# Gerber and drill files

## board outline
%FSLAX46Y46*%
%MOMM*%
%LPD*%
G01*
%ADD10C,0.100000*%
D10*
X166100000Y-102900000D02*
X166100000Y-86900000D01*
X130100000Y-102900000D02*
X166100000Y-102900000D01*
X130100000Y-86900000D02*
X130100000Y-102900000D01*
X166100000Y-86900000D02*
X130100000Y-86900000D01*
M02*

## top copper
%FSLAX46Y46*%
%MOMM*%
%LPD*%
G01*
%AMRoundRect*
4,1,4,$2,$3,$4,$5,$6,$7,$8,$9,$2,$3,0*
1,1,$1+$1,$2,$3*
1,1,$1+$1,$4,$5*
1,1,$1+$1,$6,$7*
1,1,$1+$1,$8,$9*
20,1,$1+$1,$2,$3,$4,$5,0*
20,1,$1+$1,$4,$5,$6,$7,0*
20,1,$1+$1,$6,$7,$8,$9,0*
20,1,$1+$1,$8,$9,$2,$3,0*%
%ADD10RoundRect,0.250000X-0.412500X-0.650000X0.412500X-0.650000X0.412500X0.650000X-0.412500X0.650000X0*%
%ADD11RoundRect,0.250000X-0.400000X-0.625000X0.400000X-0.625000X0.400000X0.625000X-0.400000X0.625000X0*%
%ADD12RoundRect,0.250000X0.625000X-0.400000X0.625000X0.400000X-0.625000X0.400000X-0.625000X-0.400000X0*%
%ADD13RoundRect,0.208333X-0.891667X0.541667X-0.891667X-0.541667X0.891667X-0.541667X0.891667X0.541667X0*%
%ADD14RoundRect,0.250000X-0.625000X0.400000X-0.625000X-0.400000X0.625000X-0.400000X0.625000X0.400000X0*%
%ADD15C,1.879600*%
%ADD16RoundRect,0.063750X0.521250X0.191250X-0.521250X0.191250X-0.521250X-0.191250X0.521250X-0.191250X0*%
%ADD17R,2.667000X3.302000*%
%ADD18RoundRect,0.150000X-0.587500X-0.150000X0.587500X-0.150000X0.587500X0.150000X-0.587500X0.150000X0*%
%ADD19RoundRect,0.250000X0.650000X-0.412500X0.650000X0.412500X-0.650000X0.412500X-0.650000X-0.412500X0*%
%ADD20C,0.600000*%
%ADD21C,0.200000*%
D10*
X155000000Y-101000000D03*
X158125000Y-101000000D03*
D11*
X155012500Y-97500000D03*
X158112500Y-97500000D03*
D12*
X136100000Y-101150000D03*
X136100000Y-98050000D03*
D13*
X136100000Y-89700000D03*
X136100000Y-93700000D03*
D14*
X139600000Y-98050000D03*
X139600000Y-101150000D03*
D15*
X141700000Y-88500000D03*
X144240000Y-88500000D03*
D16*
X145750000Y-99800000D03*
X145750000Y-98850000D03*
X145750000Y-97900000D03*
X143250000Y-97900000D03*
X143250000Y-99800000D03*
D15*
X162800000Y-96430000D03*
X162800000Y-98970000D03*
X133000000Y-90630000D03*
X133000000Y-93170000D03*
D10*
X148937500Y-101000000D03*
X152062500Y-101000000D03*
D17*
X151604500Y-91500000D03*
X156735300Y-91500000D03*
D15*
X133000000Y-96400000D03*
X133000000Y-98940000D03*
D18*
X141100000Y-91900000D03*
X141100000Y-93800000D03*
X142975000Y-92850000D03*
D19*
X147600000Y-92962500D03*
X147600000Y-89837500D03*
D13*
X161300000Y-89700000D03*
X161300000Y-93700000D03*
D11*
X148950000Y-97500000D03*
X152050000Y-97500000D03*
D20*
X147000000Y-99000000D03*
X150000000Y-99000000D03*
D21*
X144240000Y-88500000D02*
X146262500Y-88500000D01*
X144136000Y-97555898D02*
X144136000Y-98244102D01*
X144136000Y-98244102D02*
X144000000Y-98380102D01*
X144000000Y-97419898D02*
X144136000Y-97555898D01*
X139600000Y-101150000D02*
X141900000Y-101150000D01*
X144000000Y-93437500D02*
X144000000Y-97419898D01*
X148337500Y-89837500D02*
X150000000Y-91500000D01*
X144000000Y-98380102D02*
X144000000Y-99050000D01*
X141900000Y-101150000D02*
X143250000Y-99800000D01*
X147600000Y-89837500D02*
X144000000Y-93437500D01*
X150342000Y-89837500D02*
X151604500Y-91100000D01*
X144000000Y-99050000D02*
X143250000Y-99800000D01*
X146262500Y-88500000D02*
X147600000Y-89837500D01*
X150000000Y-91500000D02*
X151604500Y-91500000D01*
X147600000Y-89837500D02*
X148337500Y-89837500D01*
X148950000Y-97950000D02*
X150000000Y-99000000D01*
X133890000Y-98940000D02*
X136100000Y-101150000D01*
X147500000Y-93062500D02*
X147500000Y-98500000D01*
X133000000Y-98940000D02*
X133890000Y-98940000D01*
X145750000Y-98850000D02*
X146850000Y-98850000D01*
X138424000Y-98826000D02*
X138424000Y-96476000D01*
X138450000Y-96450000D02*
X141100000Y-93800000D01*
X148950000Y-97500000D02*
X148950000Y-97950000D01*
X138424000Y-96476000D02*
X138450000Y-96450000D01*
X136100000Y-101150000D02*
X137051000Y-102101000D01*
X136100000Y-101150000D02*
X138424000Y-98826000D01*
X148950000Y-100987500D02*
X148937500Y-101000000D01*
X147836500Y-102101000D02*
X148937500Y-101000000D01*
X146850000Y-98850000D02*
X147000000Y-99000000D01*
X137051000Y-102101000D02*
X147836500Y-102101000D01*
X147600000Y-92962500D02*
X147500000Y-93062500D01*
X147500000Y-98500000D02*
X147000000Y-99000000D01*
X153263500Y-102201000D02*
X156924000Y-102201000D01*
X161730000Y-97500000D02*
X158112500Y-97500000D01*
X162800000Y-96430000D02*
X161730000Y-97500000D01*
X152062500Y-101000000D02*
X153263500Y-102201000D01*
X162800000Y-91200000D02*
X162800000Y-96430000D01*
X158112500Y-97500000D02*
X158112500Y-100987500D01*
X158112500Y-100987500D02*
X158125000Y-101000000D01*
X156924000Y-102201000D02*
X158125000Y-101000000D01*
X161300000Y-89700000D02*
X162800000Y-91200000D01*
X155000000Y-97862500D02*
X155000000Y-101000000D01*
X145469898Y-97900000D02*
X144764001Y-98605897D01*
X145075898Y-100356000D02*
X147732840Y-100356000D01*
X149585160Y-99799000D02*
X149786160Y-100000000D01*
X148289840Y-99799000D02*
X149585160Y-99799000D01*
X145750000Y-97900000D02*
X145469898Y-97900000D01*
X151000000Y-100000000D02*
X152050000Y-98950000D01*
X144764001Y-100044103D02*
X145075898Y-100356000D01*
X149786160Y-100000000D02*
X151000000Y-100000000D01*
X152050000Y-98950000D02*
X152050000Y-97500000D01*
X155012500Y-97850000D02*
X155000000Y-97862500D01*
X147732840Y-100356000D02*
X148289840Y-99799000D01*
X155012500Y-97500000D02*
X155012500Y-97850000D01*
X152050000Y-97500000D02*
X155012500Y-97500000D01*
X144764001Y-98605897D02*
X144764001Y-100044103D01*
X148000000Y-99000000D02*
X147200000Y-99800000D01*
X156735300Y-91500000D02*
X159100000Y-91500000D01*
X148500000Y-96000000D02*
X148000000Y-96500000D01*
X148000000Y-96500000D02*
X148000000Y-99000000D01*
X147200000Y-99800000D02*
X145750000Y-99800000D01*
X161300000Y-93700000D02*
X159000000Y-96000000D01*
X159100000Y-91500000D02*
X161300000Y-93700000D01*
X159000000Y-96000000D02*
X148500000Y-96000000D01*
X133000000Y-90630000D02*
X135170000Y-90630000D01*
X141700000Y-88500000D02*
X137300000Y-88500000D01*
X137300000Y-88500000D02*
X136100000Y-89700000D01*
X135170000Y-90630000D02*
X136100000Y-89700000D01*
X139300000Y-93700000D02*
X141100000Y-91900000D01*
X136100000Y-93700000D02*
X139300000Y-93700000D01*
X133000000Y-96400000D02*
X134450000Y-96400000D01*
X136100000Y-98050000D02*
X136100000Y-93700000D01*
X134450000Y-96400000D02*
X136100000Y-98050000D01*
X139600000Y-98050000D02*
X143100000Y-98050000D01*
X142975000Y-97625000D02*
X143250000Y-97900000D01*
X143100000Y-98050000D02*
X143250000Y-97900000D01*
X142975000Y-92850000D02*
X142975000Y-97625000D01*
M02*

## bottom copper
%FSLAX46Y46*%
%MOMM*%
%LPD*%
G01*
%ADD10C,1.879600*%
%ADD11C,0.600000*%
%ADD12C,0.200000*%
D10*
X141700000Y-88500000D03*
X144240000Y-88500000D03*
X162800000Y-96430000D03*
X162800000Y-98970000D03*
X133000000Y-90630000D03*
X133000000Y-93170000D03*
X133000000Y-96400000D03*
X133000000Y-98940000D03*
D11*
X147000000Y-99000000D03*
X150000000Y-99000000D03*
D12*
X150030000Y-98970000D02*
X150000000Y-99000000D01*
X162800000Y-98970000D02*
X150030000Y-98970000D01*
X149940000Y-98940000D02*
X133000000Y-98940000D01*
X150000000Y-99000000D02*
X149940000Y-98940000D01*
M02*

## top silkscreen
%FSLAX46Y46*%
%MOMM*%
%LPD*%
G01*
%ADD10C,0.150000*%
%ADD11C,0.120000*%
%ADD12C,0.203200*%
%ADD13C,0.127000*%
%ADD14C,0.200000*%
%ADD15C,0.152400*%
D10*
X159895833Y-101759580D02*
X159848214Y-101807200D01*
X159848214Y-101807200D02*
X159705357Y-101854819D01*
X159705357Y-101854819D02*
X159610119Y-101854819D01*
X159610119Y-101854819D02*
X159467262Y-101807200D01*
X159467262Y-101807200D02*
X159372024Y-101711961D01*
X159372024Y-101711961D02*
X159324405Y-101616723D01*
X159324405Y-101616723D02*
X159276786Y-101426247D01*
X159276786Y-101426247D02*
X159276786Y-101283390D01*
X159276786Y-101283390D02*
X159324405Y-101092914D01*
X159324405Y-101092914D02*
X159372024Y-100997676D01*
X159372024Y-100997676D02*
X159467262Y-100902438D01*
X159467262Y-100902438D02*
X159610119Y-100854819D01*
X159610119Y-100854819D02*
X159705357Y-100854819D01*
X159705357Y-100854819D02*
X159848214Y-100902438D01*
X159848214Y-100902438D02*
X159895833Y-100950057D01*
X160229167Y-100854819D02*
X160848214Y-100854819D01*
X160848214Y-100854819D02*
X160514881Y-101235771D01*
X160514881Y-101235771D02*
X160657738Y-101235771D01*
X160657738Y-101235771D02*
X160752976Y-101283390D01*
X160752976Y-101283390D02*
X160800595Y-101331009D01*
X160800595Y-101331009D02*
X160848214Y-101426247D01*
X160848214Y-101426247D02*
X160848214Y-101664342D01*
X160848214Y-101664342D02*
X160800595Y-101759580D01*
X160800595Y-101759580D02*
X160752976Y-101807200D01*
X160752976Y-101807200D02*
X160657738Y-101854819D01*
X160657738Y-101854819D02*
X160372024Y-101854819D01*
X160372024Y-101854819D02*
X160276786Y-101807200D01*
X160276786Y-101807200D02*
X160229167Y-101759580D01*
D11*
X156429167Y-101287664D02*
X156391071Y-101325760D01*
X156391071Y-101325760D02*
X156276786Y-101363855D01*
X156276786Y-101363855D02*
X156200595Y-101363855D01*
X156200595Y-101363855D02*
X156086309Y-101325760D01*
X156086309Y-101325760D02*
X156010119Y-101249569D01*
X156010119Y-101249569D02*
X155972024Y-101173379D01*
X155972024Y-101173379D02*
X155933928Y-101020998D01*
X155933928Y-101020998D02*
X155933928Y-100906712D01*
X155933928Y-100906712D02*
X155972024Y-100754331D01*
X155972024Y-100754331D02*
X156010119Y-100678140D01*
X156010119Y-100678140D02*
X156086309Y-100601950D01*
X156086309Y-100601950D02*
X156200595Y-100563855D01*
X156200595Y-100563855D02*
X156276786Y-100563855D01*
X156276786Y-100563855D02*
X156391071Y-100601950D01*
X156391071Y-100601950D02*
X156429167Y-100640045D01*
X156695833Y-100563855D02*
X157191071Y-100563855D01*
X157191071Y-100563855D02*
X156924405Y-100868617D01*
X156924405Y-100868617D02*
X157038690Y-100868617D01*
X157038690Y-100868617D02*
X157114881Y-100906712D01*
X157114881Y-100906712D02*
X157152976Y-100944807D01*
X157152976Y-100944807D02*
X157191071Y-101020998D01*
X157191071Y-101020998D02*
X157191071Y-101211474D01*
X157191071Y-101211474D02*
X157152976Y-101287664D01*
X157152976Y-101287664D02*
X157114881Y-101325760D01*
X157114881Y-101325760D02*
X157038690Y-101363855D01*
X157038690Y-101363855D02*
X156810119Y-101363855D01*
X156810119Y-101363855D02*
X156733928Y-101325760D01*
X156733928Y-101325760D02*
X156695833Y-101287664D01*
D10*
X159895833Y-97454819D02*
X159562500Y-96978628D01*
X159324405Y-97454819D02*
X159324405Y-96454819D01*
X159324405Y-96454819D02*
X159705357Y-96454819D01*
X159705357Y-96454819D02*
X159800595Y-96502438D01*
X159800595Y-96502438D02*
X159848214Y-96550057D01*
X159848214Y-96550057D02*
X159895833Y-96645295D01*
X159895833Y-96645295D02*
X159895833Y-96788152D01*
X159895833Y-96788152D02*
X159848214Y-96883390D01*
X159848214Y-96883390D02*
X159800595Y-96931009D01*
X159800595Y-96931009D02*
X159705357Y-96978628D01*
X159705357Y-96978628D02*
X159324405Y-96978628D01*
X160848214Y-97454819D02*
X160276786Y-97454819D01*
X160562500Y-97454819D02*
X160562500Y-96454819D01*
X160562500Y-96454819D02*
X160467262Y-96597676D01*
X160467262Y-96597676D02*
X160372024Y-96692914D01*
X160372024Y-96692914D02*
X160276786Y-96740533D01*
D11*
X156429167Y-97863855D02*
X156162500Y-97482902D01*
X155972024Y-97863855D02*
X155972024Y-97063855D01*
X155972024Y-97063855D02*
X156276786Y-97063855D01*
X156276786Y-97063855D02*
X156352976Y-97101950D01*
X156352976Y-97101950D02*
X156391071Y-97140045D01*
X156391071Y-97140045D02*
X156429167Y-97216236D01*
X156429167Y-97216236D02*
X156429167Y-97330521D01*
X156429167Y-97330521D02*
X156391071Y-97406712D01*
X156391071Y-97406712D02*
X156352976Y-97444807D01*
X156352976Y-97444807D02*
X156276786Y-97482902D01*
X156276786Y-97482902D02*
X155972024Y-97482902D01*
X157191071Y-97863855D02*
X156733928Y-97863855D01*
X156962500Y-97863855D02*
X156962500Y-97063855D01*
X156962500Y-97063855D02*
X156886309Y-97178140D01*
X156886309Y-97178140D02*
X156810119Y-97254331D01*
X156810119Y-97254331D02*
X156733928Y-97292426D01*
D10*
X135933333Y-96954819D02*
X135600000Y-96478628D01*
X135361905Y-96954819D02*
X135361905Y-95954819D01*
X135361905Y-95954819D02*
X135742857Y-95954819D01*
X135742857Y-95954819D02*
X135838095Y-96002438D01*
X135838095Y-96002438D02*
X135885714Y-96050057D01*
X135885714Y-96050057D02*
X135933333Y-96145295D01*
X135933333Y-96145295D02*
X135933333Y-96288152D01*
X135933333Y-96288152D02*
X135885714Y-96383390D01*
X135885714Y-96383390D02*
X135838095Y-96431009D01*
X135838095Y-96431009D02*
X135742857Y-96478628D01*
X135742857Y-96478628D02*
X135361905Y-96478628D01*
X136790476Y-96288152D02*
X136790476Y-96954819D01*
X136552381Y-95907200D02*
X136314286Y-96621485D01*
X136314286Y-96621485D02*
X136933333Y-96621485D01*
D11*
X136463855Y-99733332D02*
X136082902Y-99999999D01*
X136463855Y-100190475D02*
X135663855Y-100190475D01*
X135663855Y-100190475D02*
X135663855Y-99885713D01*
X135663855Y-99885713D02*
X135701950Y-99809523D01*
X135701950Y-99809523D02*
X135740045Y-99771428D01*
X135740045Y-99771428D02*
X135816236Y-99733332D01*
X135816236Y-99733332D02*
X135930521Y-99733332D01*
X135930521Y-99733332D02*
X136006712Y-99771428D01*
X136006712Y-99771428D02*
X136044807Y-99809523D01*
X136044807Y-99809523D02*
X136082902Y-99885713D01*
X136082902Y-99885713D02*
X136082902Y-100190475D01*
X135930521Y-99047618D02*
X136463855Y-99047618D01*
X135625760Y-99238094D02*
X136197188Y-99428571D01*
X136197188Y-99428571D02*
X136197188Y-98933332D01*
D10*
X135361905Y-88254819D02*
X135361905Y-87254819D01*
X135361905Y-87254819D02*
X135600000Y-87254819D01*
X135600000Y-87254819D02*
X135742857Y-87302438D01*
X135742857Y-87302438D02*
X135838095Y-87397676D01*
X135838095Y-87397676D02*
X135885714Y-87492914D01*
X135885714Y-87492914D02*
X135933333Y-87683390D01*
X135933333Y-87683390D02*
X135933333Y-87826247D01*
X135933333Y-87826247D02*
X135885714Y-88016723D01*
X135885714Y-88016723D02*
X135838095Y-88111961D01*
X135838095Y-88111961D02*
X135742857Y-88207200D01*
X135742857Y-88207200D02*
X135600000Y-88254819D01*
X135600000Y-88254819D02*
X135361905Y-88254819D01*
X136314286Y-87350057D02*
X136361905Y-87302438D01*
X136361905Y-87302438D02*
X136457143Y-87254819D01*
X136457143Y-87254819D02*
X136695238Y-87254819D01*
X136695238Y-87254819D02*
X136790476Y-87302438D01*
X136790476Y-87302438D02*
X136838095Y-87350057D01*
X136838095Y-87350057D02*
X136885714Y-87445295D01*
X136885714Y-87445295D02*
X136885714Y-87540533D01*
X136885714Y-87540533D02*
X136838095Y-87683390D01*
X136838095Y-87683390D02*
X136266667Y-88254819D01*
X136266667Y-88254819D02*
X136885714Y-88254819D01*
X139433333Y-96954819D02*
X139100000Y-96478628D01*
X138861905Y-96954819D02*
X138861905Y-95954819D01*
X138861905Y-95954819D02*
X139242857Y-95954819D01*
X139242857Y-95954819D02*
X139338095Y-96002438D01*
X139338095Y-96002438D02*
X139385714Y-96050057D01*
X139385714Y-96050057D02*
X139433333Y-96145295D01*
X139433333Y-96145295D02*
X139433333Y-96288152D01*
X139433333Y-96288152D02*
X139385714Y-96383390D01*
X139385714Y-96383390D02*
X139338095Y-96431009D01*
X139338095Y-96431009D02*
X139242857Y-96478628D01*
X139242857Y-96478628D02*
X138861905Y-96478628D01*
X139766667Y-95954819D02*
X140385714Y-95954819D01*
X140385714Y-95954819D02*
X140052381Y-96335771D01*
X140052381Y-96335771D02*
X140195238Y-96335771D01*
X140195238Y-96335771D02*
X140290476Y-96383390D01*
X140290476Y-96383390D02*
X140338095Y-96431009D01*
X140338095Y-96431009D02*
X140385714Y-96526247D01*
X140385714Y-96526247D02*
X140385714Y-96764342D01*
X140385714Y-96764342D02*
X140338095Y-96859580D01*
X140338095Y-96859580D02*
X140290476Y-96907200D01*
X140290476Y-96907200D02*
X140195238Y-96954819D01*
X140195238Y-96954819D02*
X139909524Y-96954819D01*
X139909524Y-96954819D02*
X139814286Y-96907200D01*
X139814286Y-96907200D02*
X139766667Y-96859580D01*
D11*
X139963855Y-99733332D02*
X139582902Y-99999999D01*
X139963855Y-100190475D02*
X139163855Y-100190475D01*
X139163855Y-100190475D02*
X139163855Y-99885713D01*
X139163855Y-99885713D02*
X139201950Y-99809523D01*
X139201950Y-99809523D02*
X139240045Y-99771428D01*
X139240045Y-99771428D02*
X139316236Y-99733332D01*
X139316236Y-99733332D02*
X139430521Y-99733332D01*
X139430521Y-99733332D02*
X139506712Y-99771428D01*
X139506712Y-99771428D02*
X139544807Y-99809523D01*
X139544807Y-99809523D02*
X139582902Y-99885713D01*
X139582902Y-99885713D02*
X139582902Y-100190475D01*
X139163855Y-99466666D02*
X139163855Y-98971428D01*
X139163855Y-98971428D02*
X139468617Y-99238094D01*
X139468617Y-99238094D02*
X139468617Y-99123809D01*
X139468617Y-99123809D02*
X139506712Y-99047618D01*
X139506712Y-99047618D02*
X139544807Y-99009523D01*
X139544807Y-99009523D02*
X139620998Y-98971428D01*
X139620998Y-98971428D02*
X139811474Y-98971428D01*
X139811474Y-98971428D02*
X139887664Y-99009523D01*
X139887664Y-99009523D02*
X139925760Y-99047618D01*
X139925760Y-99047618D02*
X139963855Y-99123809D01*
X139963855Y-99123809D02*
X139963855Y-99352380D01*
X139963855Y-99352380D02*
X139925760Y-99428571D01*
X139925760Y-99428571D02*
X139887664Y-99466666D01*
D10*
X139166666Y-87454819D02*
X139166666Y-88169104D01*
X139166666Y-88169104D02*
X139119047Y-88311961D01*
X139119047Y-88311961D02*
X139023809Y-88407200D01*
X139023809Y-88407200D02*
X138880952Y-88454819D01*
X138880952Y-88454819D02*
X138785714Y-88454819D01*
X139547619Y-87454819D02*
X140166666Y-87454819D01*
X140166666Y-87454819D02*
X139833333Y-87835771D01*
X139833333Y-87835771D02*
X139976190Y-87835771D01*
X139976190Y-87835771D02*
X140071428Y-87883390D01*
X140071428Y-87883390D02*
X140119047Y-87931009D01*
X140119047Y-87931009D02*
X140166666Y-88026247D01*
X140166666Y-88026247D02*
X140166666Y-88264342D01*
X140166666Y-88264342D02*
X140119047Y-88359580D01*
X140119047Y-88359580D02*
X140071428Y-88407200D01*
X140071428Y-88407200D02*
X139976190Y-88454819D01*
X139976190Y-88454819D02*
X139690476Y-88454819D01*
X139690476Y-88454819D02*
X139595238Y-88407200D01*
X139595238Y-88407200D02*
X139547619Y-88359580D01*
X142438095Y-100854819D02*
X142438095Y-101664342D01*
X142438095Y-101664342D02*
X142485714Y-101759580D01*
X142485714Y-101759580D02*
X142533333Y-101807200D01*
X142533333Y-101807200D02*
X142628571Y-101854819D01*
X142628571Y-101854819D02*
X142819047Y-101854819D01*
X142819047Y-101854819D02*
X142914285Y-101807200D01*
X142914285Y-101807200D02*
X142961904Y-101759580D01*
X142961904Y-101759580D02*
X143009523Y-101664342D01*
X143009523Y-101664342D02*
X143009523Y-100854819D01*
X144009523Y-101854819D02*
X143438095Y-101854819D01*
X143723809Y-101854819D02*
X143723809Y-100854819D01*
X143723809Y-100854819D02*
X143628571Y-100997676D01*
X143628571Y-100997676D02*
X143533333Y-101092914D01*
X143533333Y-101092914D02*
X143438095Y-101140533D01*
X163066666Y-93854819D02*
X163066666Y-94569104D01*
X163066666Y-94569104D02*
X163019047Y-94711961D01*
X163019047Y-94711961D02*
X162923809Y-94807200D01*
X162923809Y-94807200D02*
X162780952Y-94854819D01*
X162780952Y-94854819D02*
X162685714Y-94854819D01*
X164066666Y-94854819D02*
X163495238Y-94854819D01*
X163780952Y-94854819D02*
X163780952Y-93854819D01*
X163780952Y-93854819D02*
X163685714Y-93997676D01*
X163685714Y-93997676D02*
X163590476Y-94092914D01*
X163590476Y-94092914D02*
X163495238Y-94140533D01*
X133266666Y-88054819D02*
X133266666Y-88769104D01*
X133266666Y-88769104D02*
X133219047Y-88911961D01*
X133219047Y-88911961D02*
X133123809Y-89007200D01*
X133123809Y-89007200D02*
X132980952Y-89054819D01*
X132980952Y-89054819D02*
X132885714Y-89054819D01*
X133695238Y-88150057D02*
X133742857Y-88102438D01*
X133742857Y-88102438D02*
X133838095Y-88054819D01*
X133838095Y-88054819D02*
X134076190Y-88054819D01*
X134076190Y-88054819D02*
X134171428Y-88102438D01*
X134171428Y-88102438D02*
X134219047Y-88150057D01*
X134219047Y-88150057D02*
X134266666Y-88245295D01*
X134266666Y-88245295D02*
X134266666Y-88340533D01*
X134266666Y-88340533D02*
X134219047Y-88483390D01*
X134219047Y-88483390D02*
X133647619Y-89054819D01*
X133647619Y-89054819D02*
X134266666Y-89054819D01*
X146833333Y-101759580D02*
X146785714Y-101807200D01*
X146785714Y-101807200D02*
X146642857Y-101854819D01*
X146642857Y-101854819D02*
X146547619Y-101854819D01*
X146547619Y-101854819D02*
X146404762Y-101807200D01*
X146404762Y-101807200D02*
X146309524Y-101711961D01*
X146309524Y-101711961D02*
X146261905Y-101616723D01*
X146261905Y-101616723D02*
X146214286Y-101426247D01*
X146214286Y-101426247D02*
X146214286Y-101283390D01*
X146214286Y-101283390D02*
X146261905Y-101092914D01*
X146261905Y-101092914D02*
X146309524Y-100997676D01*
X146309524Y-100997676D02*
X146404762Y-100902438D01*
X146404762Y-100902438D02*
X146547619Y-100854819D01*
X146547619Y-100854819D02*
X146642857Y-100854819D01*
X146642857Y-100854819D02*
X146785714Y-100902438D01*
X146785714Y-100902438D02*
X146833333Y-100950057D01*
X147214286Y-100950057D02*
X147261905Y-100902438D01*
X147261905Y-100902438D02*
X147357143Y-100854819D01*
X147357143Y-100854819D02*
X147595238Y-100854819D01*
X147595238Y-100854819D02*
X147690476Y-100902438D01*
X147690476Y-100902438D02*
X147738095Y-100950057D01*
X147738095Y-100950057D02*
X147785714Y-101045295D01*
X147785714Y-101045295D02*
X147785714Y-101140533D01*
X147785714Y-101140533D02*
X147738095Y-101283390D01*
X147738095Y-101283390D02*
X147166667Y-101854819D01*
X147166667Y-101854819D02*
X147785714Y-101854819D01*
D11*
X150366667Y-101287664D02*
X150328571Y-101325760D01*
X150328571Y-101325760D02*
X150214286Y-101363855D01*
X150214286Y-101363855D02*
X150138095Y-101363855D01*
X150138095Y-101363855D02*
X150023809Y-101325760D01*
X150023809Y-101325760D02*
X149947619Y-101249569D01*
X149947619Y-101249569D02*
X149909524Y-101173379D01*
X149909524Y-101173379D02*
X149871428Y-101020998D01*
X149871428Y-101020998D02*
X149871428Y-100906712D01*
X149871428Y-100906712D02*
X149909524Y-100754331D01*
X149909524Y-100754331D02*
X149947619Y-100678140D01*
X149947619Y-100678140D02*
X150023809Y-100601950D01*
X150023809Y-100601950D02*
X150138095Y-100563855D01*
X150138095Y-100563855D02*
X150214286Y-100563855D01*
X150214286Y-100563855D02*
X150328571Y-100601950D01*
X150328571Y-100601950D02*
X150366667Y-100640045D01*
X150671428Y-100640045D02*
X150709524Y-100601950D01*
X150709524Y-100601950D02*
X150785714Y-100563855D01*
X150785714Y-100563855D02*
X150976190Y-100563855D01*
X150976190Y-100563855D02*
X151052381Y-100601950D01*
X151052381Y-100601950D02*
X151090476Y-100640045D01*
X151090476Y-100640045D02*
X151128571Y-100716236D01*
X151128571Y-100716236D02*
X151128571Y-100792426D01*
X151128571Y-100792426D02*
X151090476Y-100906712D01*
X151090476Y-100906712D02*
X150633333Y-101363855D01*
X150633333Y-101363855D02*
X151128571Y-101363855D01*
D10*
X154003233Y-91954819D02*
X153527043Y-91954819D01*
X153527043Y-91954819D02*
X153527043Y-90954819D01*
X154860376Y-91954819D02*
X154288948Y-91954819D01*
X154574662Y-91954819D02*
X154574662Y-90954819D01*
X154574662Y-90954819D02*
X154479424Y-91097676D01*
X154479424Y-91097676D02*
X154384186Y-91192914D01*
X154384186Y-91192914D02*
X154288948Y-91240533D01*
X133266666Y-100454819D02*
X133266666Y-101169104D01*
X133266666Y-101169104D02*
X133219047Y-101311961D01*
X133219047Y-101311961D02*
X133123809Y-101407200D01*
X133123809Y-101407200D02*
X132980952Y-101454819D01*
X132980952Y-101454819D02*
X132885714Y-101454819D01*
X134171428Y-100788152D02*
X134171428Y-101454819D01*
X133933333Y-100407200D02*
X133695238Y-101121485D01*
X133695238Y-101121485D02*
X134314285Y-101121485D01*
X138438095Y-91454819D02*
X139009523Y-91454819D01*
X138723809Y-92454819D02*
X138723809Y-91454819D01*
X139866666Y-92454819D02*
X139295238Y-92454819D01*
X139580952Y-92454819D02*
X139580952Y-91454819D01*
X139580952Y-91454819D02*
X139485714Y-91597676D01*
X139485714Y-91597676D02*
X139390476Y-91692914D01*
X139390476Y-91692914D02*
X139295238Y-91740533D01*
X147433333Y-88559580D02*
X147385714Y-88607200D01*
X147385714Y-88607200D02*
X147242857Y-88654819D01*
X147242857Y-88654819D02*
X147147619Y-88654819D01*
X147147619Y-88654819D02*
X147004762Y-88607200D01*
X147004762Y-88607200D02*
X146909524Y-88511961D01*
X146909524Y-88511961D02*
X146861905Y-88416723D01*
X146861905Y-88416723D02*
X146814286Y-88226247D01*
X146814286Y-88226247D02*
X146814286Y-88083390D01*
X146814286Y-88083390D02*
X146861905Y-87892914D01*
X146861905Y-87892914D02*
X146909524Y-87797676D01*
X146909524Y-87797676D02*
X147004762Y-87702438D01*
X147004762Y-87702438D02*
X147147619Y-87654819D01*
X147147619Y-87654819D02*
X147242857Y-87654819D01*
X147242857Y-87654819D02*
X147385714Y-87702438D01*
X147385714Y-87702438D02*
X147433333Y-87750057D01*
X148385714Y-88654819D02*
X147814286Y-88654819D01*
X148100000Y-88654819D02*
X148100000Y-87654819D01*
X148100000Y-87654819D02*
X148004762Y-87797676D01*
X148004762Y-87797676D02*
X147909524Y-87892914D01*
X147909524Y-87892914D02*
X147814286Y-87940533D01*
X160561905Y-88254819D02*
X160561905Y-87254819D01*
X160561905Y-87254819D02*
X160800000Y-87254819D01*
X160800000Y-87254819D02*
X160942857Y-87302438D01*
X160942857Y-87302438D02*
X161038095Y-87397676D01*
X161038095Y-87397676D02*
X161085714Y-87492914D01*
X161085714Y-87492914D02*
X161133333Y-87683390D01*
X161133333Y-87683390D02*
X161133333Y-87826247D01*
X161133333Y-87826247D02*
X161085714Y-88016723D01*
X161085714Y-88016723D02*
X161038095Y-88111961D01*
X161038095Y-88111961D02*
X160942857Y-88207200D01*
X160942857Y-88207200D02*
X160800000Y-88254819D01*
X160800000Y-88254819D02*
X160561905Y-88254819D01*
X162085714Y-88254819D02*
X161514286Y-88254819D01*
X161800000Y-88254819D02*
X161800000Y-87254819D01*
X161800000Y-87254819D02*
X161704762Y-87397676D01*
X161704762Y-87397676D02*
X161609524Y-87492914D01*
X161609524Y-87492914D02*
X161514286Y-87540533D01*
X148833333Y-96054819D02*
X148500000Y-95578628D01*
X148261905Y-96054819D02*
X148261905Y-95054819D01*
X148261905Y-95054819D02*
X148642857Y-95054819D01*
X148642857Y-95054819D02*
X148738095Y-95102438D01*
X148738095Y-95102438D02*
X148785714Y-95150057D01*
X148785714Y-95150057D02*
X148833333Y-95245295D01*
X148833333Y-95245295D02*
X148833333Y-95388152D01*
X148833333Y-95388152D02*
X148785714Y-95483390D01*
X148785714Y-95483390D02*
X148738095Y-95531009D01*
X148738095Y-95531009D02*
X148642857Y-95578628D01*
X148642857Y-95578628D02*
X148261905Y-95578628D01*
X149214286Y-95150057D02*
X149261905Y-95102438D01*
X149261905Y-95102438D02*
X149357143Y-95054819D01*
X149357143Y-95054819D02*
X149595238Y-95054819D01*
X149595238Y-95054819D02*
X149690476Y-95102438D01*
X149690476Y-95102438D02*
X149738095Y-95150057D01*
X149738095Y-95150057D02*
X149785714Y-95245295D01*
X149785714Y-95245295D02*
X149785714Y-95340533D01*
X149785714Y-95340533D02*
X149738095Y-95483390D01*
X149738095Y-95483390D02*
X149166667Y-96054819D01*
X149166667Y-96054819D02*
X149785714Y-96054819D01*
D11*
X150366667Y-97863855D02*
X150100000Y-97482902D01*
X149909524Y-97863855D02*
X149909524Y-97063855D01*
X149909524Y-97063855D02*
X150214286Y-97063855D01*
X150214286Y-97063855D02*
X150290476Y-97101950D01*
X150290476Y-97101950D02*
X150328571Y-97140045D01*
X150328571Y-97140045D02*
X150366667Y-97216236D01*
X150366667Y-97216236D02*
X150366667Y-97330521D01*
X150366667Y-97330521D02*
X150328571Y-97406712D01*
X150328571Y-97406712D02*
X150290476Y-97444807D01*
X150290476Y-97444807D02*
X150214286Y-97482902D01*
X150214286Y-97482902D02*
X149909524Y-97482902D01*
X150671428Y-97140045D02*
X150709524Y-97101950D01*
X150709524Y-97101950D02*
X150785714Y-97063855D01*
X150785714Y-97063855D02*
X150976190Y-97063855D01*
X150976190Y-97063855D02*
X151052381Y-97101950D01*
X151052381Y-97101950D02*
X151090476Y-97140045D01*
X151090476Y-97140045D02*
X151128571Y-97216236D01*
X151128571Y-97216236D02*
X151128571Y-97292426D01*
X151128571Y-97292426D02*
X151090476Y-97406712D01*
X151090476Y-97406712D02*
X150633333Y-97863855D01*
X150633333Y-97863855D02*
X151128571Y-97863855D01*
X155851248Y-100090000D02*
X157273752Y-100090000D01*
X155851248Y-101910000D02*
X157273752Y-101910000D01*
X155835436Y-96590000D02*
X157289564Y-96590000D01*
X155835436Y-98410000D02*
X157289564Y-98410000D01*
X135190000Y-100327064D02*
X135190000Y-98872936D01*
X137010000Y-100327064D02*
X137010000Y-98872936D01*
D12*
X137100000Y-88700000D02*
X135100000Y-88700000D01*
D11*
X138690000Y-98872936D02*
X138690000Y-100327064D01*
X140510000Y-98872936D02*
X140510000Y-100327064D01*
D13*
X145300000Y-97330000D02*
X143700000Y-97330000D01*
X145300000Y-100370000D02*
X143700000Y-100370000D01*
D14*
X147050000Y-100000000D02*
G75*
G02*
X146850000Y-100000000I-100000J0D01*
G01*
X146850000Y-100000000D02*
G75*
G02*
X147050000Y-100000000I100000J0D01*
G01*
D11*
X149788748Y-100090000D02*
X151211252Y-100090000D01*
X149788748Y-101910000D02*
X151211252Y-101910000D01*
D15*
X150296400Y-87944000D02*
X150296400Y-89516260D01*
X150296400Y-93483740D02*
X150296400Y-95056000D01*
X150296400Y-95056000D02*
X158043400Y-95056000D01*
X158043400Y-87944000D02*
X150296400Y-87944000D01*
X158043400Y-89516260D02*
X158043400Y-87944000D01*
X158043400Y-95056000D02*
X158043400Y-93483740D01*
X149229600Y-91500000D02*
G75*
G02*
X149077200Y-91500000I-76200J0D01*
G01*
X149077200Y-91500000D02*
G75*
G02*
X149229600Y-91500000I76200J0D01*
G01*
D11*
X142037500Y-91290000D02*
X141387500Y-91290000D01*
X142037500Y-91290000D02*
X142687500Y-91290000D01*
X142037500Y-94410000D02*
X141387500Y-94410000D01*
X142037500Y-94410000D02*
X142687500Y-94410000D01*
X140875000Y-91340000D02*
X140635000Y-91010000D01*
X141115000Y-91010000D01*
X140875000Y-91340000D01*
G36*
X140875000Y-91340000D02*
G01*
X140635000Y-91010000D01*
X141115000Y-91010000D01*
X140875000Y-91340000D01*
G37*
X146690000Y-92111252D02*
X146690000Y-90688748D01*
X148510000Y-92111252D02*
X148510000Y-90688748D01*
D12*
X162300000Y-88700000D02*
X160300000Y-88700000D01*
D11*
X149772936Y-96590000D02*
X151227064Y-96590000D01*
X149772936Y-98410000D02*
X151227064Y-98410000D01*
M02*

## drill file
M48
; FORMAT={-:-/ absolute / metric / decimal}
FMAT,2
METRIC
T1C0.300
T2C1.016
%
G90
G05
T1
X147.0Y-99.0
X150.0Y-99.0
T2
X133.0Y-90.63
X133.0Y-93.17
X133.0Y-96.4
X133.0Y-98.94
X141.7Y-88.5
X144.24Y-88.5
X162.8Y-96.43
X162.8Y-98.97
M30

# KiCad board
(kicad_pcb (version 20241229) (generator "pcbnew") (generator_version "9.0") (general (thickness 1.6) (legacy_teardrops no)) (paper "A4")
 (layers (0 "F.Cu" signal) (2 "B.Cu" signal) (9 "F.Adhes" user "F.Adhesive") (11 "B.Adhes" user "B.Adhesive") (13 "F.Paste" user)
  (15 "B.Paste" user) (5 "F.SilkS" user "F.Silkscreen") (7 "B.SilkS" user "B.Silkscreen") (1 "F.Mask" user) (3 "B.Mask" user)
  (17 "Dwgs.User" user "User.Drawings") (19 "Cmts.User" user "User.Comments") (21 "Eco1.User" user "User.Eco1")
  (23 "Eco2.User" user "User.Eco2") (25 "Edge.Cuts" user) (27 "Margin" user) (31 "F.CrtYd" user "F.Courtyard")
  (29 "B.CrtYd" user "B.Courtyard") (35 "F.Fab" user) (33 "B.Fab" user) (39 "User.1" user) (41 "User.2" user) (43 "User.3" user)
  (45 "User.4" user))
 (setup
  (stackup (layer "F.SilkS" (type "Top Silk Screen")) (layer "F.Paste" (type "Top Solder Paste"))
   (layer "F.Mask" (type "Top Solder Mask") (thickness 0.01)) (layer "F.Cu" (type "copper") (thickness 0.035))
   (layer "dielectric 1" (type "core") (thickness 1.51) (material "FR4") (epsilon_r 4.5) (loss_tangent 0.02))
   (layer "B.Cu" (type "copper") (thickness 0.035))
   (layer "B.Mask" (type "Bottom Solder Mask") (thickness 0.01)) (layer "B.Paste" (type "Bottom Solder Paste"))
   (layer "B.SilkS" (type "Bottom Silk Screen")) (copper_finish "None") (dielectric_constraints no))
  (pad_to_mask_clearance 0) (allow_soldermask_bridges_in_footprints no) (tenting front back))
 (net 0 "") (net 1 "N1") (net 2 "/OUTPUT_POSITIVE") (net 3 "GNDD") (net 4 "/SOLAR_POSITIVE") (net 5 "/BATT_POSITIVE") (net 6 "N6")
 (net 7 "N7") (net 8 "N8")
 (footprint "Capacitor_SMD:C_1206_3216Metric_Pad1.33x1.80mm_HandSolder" (layer "F.Cu") (at 156.5625 101)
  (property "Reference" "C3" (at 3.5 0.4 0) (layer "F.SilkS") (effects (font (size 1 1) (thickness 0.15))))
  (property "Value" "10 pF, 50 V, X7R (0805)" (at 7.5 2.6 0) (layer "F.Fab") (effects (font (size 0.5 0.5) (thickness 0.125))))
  (fp_line (start -0.711252 -0.91) (end 0.711252 -0.91) (stroke (width 0.12) (type solid)) (layer "F.SilkS"))
  (fp_line (start -0.711252 0.91) (end 0.711252 0.91) (stroke (width 0.12) (type solid)) (layer "F.SilkS"))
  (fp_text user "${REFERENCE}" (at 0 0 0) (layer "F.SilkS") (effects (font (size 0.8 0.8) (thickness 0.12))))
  (pad "1" smd roundrect (at -1.5625 0) (size 1.325 1.8) (layers "F.Cu" "F.Mask" "F.Paste") (roundrect_rratio 0.188679) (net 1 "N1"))
  (pad "2" smd roundrect (at 1.5625 0) (size 1.325 1.8) (layers "F.Cu" "F.Mask" "F.Paste") (roundrect_rratio 0.188679)
   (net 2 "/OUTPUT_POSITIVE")))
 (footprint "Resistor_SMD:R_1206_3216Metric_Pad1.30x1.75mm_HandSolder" (layer "F.Cu") (at 156.5625 97.5)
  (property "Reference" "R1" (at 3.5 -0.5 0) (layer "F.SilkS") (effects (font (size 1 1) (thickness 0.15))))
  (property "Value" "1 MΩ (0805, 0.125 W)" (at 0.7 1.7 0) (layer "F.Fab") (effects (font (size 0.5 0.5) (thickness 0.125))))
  (fp_line (start -0.727064 -0.91) (end 0.727064 -0.91) (stroke (width 0.12) (type solid)) (layer "F.SilkS"))
  (fp_line (start -0.727064 0.91) (end 0.727064 0.91) (stroke (width 0.12) (type solid)) (layer "F.SilkS"))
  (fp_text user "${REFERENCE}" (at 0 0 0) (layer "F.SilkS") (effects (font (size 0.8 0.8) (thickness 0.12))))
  (pad "1" smd roundrect (at -1.55 0) (size 1.3 1.75) (layers "F.Cu" "F.Mask" "F.Paste") (roundrect_rratio 0.192308) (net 1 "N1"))
  (pad "2" smd roundrect (at 1.55 0) (size 1.3 1.75) (layers "F.Cu" "F.Mask" "F.Paste") (roundrect_rratio 0.192308)
   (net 2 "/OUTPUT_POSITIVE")))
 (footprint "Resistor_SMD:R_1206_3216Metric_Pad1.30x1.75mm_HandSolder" (layer "F.Cu") (at 136.1 99.6 90)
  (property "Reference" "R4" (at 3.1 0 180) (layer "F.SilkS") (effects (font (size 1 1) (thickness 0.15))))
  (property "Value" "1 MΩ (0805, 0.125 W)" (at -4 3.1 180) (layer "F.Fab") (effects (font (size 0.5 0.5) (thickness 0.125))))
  (fp_line (start -0.727064 -0.91) (end 0.727064 -0.91) (stroke (width 0.12) (type solid)) (layer "F.SilkS"))
  (fp_line (start -0.727064 0.91) (end 0.727064 0.91) (stroke (width 0.12) (type solid)) (layer "F.SilkS"))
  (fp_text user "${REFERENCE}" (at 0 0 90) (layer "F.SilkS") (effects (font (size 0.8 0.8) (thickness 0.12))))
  (pad "1" smd roundrect (at -1.55 0 90) (size 1.3 1.75) (layers "F.Cu" "F.Mask" "F.Paste") (roundrect_rratio 0.192308) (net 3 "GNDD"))
  (pad "2" smd roundrect (at 1.55 0 90) (size 1.3 1.75) (layers "F.Cu" "F.Mask" "F.Paste") (roundrect_rratio 0.192308)
   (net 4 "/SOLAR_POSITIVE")))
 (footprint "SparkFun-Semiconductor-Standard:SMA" (layer "F.Cu") (at 136.1 91.7 -90)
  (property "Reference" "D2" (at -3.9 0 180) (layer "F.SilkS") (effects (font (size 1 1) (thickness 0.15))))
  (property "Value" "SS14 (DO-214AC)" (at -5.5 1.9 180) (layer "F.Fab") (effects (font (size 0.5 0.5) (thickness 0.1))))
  (fp_line (start -3 -1) (end -3 1) (stroke (width 0.2032) (type solid)) (layer "F.SilkS"))
  (pad "1" smd roundrect (at -2 0 270) (size 1.5 2.2) (layers "F.Cu" "F.Mask" "F.Paste") (roundrect_rratio 0.1388888889)
   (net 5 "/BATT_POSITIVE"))
  (pad "2" smd roundrect (at 2 0 270) (size 1.5 2.2) (layers "F.Cu" "F.Mask" "F.Paste") (roundrect_rratio 0.1388888889)
   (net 4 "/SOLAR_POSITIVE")))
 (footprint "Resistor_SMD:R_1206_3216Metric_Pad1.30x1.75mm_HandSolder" (layer "F.Cu") (at 139.6 99.6 -90)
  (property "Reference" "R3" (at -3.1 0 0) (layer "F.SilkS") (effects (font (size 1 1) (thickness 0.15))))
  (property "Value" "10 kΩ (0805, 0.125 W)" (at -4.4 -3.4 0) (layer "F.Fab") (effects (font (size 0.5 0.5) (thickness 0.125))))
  (fp_line (start -0.727064 0.91) (end 0.727064 0.91) (stroke (width 0.12) (type solid)) (layer "F.SilkS"))
  (fp_line (start -0.727064 -0.91) (end 0.727064 -0.91) (stroke (width 0.12) (type solid)) (layer "F.SilkS"))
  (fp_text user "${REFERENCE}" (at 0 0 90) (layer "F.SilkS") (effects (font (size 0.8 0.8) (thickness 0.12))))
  (pad "1" smd roundrect (at -1.55 0 270) (size 1.3 1.75) (layers "F.Cu" "F.Mask" "F.Paste") (roundrect_rratio 0.192308) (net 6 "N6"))
  (pad "2" smd roundrect (at 1.55 0 270) (size 1.3 1.75) (layers "F.Cu" "F.Mask" "F.Paste") (roundrect_rratio 0.192308) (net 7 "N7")))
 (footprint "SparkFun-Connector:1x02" (layer "F.Cu") (at 141.7 88.5)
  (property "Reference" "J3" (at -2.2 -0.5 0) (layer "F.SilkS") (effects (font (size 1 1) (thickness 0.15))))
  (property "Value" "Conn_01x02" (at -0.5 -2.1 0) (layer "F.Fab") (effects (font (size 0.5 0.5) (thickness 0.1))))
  (pad "1" thru_hole circle (at 0 0 90) (size 1.8796 1.8796) (drill 1.016) (layers "*.Cu" "*.Mask") (remove_unused_layers yes)
   (keep_end_layers yes) (zone_layer_connections) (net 5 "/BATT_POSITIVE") (thermal_bridge_angle 0))
  (pad "2" thru_hole circle (at 2.54 0 90) (size 1.8796 1.8796) (drill 1.016) (layers "*.Cu" "*.Mask") (remove_unused_layers yes)
   (keep_end_layers yes) (zone_layer_connections) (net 7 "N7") (thermal_bridge_angle 0)))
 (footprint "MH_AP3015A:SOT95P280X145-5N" (layer "F.Cu") (at 144.5 98.85 180)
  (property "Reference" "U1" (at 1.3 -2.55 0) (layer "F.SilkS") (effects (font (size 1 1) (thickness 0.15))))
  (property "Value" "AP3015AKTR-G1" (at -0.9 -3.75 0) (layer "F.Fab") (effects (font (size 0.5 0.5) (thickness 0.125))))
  (fp_line (start -0.8 1.52) (end 0.8 1.52) (stroke (width 0.127) (type solid)) (layer "F.SilkS"))
  (fp_line (start -0.8 -1.52) (end 0.8 -1.52) (stroke (width 0.127) (type solid)) (layer "F.SilkS"))
  (fp_circle (center -2.45 -1.15) (end -2.35 -1.15) (stroke (width 0.2) (type solid)) (fill no) (layer "F.SilkS"))
  (pad "1" smd roundrect (at -1.25 -0.95 180) (size 1.17 0.51) (layers "F.Cu" "F.Mask" "F.Paste") (roundrect_rratio 0.125) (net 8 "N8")
   (solder_mask_margin 0.102))
  (pad "2" smd roundrect (at -1.25 0 180) (size 1.17 0.51) (layers "F.Cu" "F.Mask" "F.Paste") (roundrect_rratio 0.125) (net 3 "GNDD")
   (solder_mask_margin 0.102))
  (pad "3" smd roundrect (at -1.25 0.95 180) (size 1.17 0.51) (layers "F.Cu" "F.Mask" "F.Paste") (roundrect_rratio 0.125) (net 1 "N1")
   (solder_mask_margin 0.102))
  (pad "4" smd roundrect (at 1.25 0.95 180) (size 1.17 0.51) (layers "F.Cu" "F.Mask" "F.Paste") (roundrect_rratio 0.125) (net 6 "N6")
   (solder_mask_margin 0.102))
  (pad "5" smd roundrect (at 1.25 -0.95 180) (size 1.17 0.51) (layers "F.Cu" "F.Mask" "F.Paste") (roundrect_rratio 0.125) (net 7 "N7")
   (solder_mask_margin 0.102)))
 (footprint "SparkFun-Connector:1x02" (layer "F.Cu") (at 162.8 96.43 -90)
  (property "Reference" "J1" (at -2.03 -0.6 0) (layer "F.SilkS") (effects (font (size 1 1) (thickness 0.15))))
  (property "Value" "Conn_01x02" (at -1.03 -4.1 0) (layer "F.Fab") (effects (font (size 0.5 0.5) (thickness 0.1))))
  (pad "1" thru_hole circle (at 0 0) (size 1.8796 1.8796) (drill 1.016) (layers "*.Cu" "*.Mask") (remove_unused_layers yes)
   (keep_end_layers yes) (zone_layer_connections) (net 2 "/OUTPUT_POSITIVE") (thermal_bridge_angle 0))
  (pad "2" thru_hole circle (at 2.54 0) (size 1.8796 1.8796) (drill 1.016) (layers "*.Cu" "*.Mask") (remove_unused_layers yes)
   (keep_end_layers yes) (zone_layer_connections) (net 3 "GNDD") (thermal_bridge_angle 0)))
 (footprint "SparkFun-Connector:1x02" (layer "F.Cu") (at 133 90.63 -90)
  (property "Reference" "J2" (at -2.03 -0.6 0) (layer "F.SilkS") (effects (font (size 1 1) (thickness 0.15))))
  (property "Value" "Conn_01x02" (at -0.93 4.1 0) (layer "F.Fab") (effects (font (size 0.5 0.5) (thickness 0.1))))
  (pad "1" thru_hole circle (at 0 0) (size 1.8796 1.8796) (drill 1.016) (layers "*.Cu" "*.Mask") (remove_unused_layers yes)
   (keep_end_layers yes) (zone_layer_connections) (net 5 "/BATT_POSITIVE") (thermal_bridge_angle 0))
  (pad "2" thru_hole circle (at 2.54 0) (size 1.8796 1.8796) (drill 1.016) (layers "*.Cu" "*.Mask") (remove_unused_layers yes)
   (keep_end_layers yes) (zone_layer_connections) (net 3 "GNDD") (thermal_bridge_angle 0)))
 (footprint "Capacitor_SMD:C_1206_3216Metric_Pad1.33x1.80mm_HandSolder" (layer "F.Cu") (at 150.5 101)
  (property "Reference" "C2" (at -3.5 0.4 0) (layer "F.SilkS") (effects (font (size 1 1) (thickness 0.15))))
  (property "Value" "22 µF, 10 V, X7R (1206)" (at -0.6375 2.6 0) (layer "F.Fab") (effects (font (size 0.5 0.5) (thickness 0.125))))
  (fp_line (start -0.711252 -0.91) (end 0.711252 -0.91) (stroke (width 0.12) (type solid)) (layer "F.SilkS"))
  (fp_line (start -0.711252 0.91) (end 0.711252 0.91) (stroke (width 0.12) (type solid)) (layer "F.SilkS"))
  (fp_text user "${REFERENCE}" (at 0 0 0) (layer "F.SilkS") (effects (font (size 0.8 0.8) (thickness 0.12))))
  (pad "1" smd roundrect (at -1.5625 0) (size 1.325 1.8) (layers "F.Cu" "F.Mask" "F.Paste") (roundrect_rratio 0.188679) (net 3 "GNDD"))
  (pad "2" smd roundrect (at 1.5625 0) (size 1.325 1.8) (layers "F.Cu" "F.Mask" "F.Paste") (roundrect_rratio 0.188679)
   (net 2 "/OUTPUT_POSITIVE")))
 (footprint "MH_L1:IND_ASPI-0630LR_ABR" (layer "F.Cu") (at 154.1699 91.5)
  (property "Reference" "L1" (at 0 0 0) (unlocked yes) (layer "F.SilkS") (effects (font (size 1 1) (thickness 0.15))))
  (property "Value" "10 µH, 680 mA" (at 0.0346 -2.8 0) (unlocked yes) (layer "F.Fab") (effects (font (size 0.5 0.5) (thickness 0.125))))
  (fp_line (start -3.8735 -3.556) (end -3.8735 -1.98374) (stroke (width 0.1524) (type solid)) (layer "F.SilkS"))
  (fp_line (start -3.8735 1.98374) (end -3.8735 3.556) (stroke (width 0.1524) (type solid)) (layer "F.SilkS"))
  (fp_line (start -3.8735 3.556) (end 3.8735 3.556) (stroke (width 0.1524) (type solid)) (layer "F.SilkS"))
  (fp_line (start 3.8735 -3.556) (end -3.8735 -3.556) (stroke (width 0.1524) (type solid)) (layer "F.SilkS"))
  (fp_line (start 3.8735 -1.98374) (end 3.8735 -3.556) (stroke (width 0.1524) (type solid)) (layer "F.SilkS"))
  (fp_line (start 3.8735 3.556) (end 3.8735 1.98374) (stroke (width 0.1524) (type solid)) (layer "F.SilkS"))
  (fp_circle (center -5.0165 0) (end -4.9403 0) (stroke (width 0.1524) (type solid)) (fill no) (layer "F.SilkS"))
  (pad "1" smd rect (at -2.5654 0 90) (size 3.302 2.667) (layers "F.Cu" "F.Mask" "F.Paste") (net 7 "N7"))
  (pad "2" smd rect (at 2.5654 0 90) (size 3.302 2.667) (layers "F.Cu" "F.Mask" "F.Paste") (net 8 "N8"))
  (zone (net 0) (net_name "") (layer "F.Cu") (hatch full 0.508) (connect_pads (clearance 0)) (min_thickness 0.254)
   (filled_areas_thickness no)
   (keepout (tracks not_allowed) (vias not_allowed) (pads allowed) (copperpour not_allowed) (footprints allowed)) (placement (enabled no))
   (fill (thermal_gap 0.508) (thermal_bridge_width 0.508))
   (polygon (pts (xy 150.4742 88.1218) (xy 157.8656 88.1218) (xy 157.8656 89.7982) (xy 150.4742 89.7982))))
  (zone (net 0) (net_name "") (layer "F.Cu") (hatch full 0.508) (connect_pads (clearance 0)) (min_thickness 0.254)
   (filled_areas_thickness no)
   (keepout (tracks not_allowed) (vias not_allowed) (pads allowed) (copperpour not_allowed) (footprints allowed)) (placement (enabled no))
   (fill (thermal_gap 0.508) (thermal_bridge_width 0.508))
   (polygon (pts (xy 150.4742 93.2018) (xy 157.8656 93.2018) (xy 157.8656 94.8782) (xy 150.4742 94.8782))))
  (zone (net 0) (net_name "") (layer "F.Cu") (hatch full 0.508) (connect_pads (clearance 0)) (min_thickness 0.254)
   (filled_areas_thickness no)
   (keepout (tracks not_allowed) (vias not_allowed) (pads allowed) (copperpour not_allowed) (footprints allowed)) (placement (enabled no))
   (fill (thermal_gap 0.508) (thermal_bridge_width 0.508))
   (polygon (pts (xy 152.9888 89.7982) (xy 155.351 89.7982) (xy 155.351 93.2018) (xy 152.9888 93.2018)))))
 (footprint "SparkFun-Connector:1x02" (layer "F.Cu") (at 133 96.4 -90)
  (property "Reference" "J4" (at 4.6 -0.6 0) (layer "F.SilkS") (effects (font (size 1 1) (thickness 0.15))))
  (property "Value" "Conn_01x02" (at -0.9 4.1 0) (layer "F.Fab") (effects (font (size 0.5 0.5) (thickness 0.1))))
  (pad "1" thru_hole circle (at 0 0) (size 1.8796 1.8796) (drill 1.016) (layers "*.Cu" "*.Mask") (remove_unused_layers yes)
   (keep_end_layers yes) (zone_layer_connections) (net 4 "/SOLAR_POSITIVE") (thermal_bridge_angle 0))
  (pad "2" thru_hole circle (at 2.54 0) (size 1.8796 1.8796) (drill 1.016) (layers "*.Cu" "*.Mask") (remove_unused_layers yes)
   (keep_end_layers yes) (zone_layer_connections) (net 3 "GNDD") (thermal_bridge_angle 0)))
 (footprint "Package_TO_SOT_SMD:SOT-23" (layer "F.Cu") (at 142.0375 92.85)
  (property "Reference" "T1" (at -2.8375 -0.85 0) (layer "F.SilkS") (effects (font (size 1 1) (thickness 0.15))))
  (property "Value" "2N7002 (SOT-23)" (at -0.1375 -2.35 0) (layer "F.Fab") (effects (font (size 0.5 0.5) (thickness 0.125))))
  (fp_line (start 0 -1.56) (end -0.65 -1.56) (stroke (width 0.12) (type solid)) (layer "F.SilkS"))
  (fp_line (start 0 -1.56) (end 0.65 -1.56) (stroke (width 0.12) (type solid)) (layer "F.SilkS"))
  (fp_line (start 0 1.56) (end -0.65 1.56) (stroke (width 0.12) (type solid)) (layer "F.SilkS"))
  (fp_line (start 0 1.56) (end 0.65 1.56) (stroke (width 0.12) (type solid)) (layer "F.SilkS"))
  (fp_poly (pts (xy -1.1625 -1.51) (xy -1.4025 -1.84) (xy -0.9225 -1.84)) (stroke (width 0.12) (type solid)) (fill yes) (layer "F.SilkS"))
  (pad "1" smd roundrect (at -0.9375 -0.95) (size 1.475 0.6) (layers "F.Cu" "F.Mask" "F.Paste") (roundrect_rratio 0.25)
   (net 4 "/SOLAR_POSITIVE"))
  (pad "2" smd roundrect (at -0.9375 0.95) (size 1.475 0.6) (layers "F.Cu" "F.Mask" "F.Paste") (roundrect_rratio 0.25) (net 3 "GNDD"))
  (pad "3" smd roundrect (at 0.9375 0) (size 1.475 0.6) (layers "F.Cu" "F.Mask" "F.Paste") (roundrect_rratio 0.25) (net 6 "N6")))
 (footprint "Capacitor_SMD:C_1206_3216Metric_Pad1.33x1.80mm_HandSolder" (layer "F.Cu") (at 147.6 91.4 90)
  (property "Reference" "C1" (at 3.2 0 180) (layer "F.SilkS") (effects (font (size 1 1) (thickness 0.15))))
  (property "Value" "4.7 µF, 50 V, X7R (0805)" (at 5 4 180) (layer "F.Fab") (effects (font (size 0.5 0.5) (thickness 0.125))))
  (fp_line (start -0.711252 -0.91) (end 0.711252 -0.91) (stroke (width 0.12) (type solid)) (layer "F.SilkS"))
  (fp_line (start -0.711252 0.91) (end 0.711252 0.91) (stroke (width 0.12) (type solid)) (layer "F.SilkS"))
  (pad "1" smd roundrect (at -1.5625 0 90) (size 1.325 1.8) (layers "F.Cu" "F.Mask" "F.Paste") (roundrect_rratio 0.188679) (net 3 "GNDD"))
  (pad "2" smd roundrect (at 1.5625 0 90) (size 1.325 1.8) (layers "F.Cu" "F.Mask" "F.Paste") (roundrect_rratio 0.188679) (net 7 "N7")))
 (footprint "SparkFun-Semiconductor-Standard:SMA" (layer "F.Cu") (at 161.3 91.7 -90)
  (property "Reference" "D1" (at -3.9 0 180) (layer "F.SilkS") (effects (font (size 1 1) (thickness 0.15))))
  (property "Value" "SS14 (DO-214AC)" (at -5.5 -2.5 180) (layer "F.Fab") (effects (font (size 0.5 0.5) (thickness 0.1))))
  (fp_line (start -3 -1) (end -3 1) (stroke (width 0.2032) (type solid)) (layer "F.SilkS"))
  (pad "1" smd roundrect (at -2 0 270) (size 1.5 2.2) (layers "F.Cu" "F.Mask" "F.Paste") (roundrect_rratio 0.1388888889)
   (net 2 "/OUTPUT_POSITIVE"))
  (pad "2" smd roundrect (at 2 0 270) (size 1.5 2.2) (layers "F.Cu" "F.Mask" "F.Paste") (roundrect_rratio 0.1388888889) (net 8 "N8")))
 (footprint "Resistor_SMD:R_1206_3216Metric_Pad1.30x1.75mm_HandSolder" (layer "F.Cu") (at 150.5 97.5)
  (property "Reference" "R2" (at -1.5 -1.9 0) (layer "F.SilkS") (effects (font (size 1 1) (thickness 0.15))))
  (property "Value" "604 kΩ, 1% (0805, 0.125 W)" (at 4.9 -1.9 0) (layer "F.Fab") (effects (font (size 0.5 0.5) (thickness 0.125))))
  (fp_line (start -0.727064 -0.91) (end 0.727064 -0.91) (stroke (width 0.12) (type solid)) (layer "F.SilkS"))
  (fp_line (start -0.727064 0.91) (end 0.727064 0.91) (stroke (width 0.12) (type solid)) (layer "F.SilkS"))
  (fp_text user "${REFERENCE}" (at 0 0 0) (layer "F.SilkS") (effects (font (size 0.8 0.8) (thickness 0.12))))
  (pad "1" smd roundrect (at -1.55 0) (size 1.3 1.75) (layers "F.Cu" "F.Mask" "F.Paste") (roundrect_rratio 0.192308) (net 3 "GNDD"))
  (pad "2" smd roundrect (at 1.55 0) (size 1.3 1.75) (layers "F.Cu" "F.Mask" "F.Paste") (roundrect_rratio 0.192308) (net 1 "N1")))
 (gr_line (start 166.1 102.9) (end 166.1 86.9) (stroke (width 0.1) (type solid)) (layer "Edge.Cuts"))
 (gr_line (start 130.1 102.9) (end 166.1 102.9) (stroke (width 0.1) (type solid)) (layer "Edge.Cuts"))
 (gr_line (start 130.1 86.9) (end 130.1 102.9) (stroke (width 0.1) (type solid)) (layer "Edge.Cuts"))
 (gr_line (start 166.1 86.9) (end 130.1 86.9) (stroke (width 0.1) (type solid)) (layer "Edge.Cuts"))
 (segment (start 144.24 88.5) (end 146.2625 88.5) (width 0.2) (layer "F.Cu") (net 7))
 (segment (start 144.136 97.555898) (end 144.136 98.244102) (width 0.2) (layer "F.Cu") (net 7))
 (segment (start 144.136 98.244102) (end 144 98.380102) (width 0.2) (layer "F.Cu") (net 7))
 (segment (start 144 97.419898) (end 144.136 97.555898) (width 0.2) (layer "F.Cu") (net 7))
 (segment (start 139.6 101.15) (end 141.9 101.15) (width 0.2) (layer "F.Cu") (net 7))
 (segment (start 144 93.4375) (end 144 97.419898) (width 0.2) (layer "F.Cu") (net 7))
 (segment (start 148.3375 89.8375) (end 150 91.5) (width 0.2) (layer "F.Cu") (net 7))
 (segment (start 144 98.380102) (end 144 99.05) (width 0.2) (layer "F.Cu") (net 7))
 (segment (start 141.9 101.15) (end 143.25 99.8) (width 0.2) (layer "F.Cu") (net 7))
 (segment (start 147.6 89.8375) (end 144 93.4375) (width 0.2) (layer "F.Cu") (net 7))
 (segment (start 150.342 89.8375) (end 151.6045 91.1) (width 0.2) (layer "F.Cu") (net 7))
 (segment (start 144 99.05) (end 143.25 99.8) (width 0.2) (layer "F.Cu") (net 7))
 (segment (start 146.2625 88.5) (end 147.6 89.8375) (width 0.2) (layer "F.Cu") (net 7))
 (segment (start 150 91.5) (end 151.6045 91.5) (width 0.2) (layer "F.Cu") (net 7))
 (segment (start 147.6 89.8375) (end 148.3375 89.8375) (width 0.2) (layer "F.Cu") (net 7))
 (segment (start 148.95 97.95) (end 150 99) (width 0.2) (layer "F.Cu") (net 3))
 (segment (start 133.89 98.94) (end 136.1 101.15) (width 0.2) (layer "F.Cu") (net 3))
 (segment (start 147.5 93.0625) (end 147.5 98.5) (width 0.2) (layer "F.Cu") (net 3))
 (segment (start 133 98.94) (end 133.89 98.94) (width 0.2) (layer "F.Cu") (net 3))
 (segment (start 145.75 98.85) (end 146.85 98.85) (width 0.2) (layer "F.Cu") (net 3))
 (segment (start 138.424 98.826) (end 138.424 96.476) (width 0.2) (layer "F.Cu") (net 3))
 (segment (start 138.45 96.45) (end 141.1 93.8) (width 0.2) (layer "F.Cu") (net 3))
 (segment (start 148.95 97.5) (end 148.95 97.95) (width 0.2) (layer "F.Cu") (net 3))
 (segment (start 138.424 96.476) (end 138.45 96.45) (width 0.2) (layer "F.Cu") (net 3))
 (segment (start 136.1 101.15) (end 137.051 102.101) (width 0.2) (layer "F.Cu") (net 3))
 (segment (start 136.1 101.15) (end 138.424 98.826) (width 0.2) (layer "F.Cu") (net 3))
 (segment (start 148.95 100.9875) (end 148.9375 101) (width 0.2) (layer "F.Cu") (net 3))
 (segment (start 147.8365 102.101) (end 148.9375 101) (width 0.2) (layer "F.Cu") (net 3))
 (segment (start 146.85 98.85) (end 147 99) (width 0.2) (layer "F.Cu") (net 3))
 (segment (start 137.051 102.101) (end 147.8365 102.101) (width 0.2) (layer "F.Cu") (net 3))
 (segment (start 147.6 92.9625) (end 147.5 93.0625) (width 0.2) (layer "F.Cu") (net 3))
 (segment (start 147.5 98.5) (end 147 99) (width 0.2) (layer "F.Cu") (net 3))
 (via (at 147 99) (size 0.6) (drill 0.3) (layers "F.Cu" "B.Cu") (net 3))
 (via (at 150 99) (size 0.6) (drill 0.3) (layers "F.Cu" "B.Cu") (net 3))
 (segment (start 150.03 98.97) (end 150 99) (width 0.2) (layer "B.Cu") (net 3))
 (segment (start 162.8 98.97) (end 150.03 98.97) (width 0.2) (layer "B.Cu") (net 3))
 (segment (start 149.94 98.94) (end 133 98.94) (width 0.2) (layer "B.Cu") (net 3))
 (segment (start 150 99) (end 149.94 98.94) (width 0.2) (layer "B.Cu") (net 3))
 (segment (start 153.2635 102.201) (end 156.924 102.201) (width 0.2) (layer "F.Cu") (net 2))
 (segment (start 161.73 97.5) (end 158.1125 97.5) (width 0.2) (layer "F.Cu") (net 2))
 (segment (start 162.8 96.43) (end 161.73 97.5) (width 0.2) (layer "F.Cu") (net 2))
 (segment (start 152.0625 101) (end 153.2635 102.201) (width 0.2) (layer "F.Cu") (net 2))
 (segment (start 162.8 91.2) (end 162.8 96.43) (width 0.2) (layer "F.Cu") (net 2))
 (segment (start 158.1125 97.5) (end 158.1125 100.9875) (width 0.2) (layer "F.Cu") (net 2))
 (segment (start 158.1125 100.9875) (end 158.125 101) (width 0.2) (layer "F.Cu") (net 2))
 (segment (start 156.924 102.201) (end 158.125 101) (width 0.2) (layer "F.Cu") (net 2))
 (segment (start 161.3 89.7) (end 162.8 91.2) (width 0.2) (layer "F.Cu") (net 2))
 (segment (start 155 97.8625) (end 155 101) (width 0.2) (layer "F.Cu") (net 1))
 (segment (start 145.469898 97.9) (end 144.764001 98.605897) (width 0.2) (layer "F.Cu") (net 1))
 (segment (start 145.075898 100.356) (end 147.73284 100.356) (width 0.2) (layer "F.Cu") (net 1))
 (segment (start 149.58516 99.799) (end 149.78616 100) (width 0.2) (layer "F.Cu") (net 1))
 (segment (start 148.28984 99.799) (end 149.58516 99.799) (width 0.2) (layer "F.Cu") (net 1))
 (segment (start 145.75 97.9) (end 145.469898 97.9) (width 0.2) (layer "F.Cu") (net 1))
 (segment (start 151 100) (end 152.05 98.95) (width 0.2) (layer "F.Cu") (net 1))
 (segment (start 144.764001 100.044103) (end 145.075898 100.356) (width 0.2) (layer "F.Cu") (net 1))
 (segment (start 149.78616 100) (end 151 100) (width 0.2) (layer "F.Cu") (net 1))
 (segment (start 152.05 98.95) (end 152.05 97.5) (width 0.2) (layer "F.Cu") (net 1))
 (segment (start 155.0125 97.85) (end 155 97.8625) (width 0.2) (layer "F.Cu") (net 1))
 (segment (start 147.73284 100.356) (end 148.28984 99.799) (width 0.2) (layer "F.Cu") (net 1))
 (segment (start 155.0125 97.5) (end 155.0125 97.85) (width 0.2) (layer "F.Cu") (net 1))
 (segment (start 152.05 97.5) (end 155.0125 97.5) (width 0.2) (layer "F.Cu") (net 1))
 (segment (start 144.764001 98.605897) (end 144.764001 100.044103) (width 0.2) (layer "F.Cu") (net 1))
 (segment (start 148 99) (end 147.2 99.8) (width 0.2) (layer "F.Cu") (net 8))
 (segment (start 156.7353 91.5) (end 159.1 91.5) (width 0.2) (layer "F.Cu") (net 8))
 (segment (start 148.5 96) (end 148 96.5) (width 0.2) (layer "F.Cu") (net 8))
 (segment (start 148 96.5) (end 148 99) (width 0.2) (layer "F.Cu") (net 8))
 (segment (start 147.2 99.8) (end 145.75 99.8) (width 0.2) (layer "F.Cu") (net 8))
 (segment (start 161.3 93.7) (end 159 96) (width 0.2) (layer "F.Cu") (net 8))
 (segment (start 159.1 91.5) (end 161.3 93.7) (width 0.2) (layer "F.Cu") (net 8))
 (segment (start 159 96) (end 148.5 96) (width 0.2) (layer "F.Cu") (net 8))
 (segment (start 133 90.63) (end 135.17 90.63) (width 0.2) (layer "F.Cu") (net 5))
 (segment (start 141.7 88.5) (end 137.3 88.5) (width 0.2) (layer "F.Cu") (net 5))
 (segment (start 137.3 88.5) (end 136.1 89.7) (width 0.2) (layer "F.Cu") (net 5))
 (segment (start 135.17 90.63) (end 136.1 89.7) (width 0.2) (layer "F.Cu") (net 5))
 (segment (start 139.3 93.7) (end 141.1 91.9) (width 0.2) (layer "F.Cu") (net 4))
 (segment (start 136.1 93.7) (end 139.3 93.7) (width 0.2) (layer "F.Cu") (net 4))
 (segment (start 133 96.4) (end 134.45 96.4) (width 0.2) (layer "F.Cu") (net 4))
 (segment (start 136.1 98.05) (end 136.1 93.7) (width 0.2) (layer "F.Cu") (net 4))
 (segment (start 134.45 96.4) (end 136.1 98.05) (width 0.2) (layer "F.Cu") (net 4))
 (segment (start 139.6 98.05) (end 143.1 98.05) (width 0.2) (layer "F.Cu") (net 6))
 (segment (start 142.975 97.625) (end 143.25 97.9) (width 0.2) (layer "F.Cu") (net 6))
 (segment (start 143.1 98.05) (end 143.25 97.9) (width 0.2) (layer "F.Cu") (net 6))
 (segment (start 142.975 92.85) (end 142.975 97.625) (width 0.2) (layer "F.Cu") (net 6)))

